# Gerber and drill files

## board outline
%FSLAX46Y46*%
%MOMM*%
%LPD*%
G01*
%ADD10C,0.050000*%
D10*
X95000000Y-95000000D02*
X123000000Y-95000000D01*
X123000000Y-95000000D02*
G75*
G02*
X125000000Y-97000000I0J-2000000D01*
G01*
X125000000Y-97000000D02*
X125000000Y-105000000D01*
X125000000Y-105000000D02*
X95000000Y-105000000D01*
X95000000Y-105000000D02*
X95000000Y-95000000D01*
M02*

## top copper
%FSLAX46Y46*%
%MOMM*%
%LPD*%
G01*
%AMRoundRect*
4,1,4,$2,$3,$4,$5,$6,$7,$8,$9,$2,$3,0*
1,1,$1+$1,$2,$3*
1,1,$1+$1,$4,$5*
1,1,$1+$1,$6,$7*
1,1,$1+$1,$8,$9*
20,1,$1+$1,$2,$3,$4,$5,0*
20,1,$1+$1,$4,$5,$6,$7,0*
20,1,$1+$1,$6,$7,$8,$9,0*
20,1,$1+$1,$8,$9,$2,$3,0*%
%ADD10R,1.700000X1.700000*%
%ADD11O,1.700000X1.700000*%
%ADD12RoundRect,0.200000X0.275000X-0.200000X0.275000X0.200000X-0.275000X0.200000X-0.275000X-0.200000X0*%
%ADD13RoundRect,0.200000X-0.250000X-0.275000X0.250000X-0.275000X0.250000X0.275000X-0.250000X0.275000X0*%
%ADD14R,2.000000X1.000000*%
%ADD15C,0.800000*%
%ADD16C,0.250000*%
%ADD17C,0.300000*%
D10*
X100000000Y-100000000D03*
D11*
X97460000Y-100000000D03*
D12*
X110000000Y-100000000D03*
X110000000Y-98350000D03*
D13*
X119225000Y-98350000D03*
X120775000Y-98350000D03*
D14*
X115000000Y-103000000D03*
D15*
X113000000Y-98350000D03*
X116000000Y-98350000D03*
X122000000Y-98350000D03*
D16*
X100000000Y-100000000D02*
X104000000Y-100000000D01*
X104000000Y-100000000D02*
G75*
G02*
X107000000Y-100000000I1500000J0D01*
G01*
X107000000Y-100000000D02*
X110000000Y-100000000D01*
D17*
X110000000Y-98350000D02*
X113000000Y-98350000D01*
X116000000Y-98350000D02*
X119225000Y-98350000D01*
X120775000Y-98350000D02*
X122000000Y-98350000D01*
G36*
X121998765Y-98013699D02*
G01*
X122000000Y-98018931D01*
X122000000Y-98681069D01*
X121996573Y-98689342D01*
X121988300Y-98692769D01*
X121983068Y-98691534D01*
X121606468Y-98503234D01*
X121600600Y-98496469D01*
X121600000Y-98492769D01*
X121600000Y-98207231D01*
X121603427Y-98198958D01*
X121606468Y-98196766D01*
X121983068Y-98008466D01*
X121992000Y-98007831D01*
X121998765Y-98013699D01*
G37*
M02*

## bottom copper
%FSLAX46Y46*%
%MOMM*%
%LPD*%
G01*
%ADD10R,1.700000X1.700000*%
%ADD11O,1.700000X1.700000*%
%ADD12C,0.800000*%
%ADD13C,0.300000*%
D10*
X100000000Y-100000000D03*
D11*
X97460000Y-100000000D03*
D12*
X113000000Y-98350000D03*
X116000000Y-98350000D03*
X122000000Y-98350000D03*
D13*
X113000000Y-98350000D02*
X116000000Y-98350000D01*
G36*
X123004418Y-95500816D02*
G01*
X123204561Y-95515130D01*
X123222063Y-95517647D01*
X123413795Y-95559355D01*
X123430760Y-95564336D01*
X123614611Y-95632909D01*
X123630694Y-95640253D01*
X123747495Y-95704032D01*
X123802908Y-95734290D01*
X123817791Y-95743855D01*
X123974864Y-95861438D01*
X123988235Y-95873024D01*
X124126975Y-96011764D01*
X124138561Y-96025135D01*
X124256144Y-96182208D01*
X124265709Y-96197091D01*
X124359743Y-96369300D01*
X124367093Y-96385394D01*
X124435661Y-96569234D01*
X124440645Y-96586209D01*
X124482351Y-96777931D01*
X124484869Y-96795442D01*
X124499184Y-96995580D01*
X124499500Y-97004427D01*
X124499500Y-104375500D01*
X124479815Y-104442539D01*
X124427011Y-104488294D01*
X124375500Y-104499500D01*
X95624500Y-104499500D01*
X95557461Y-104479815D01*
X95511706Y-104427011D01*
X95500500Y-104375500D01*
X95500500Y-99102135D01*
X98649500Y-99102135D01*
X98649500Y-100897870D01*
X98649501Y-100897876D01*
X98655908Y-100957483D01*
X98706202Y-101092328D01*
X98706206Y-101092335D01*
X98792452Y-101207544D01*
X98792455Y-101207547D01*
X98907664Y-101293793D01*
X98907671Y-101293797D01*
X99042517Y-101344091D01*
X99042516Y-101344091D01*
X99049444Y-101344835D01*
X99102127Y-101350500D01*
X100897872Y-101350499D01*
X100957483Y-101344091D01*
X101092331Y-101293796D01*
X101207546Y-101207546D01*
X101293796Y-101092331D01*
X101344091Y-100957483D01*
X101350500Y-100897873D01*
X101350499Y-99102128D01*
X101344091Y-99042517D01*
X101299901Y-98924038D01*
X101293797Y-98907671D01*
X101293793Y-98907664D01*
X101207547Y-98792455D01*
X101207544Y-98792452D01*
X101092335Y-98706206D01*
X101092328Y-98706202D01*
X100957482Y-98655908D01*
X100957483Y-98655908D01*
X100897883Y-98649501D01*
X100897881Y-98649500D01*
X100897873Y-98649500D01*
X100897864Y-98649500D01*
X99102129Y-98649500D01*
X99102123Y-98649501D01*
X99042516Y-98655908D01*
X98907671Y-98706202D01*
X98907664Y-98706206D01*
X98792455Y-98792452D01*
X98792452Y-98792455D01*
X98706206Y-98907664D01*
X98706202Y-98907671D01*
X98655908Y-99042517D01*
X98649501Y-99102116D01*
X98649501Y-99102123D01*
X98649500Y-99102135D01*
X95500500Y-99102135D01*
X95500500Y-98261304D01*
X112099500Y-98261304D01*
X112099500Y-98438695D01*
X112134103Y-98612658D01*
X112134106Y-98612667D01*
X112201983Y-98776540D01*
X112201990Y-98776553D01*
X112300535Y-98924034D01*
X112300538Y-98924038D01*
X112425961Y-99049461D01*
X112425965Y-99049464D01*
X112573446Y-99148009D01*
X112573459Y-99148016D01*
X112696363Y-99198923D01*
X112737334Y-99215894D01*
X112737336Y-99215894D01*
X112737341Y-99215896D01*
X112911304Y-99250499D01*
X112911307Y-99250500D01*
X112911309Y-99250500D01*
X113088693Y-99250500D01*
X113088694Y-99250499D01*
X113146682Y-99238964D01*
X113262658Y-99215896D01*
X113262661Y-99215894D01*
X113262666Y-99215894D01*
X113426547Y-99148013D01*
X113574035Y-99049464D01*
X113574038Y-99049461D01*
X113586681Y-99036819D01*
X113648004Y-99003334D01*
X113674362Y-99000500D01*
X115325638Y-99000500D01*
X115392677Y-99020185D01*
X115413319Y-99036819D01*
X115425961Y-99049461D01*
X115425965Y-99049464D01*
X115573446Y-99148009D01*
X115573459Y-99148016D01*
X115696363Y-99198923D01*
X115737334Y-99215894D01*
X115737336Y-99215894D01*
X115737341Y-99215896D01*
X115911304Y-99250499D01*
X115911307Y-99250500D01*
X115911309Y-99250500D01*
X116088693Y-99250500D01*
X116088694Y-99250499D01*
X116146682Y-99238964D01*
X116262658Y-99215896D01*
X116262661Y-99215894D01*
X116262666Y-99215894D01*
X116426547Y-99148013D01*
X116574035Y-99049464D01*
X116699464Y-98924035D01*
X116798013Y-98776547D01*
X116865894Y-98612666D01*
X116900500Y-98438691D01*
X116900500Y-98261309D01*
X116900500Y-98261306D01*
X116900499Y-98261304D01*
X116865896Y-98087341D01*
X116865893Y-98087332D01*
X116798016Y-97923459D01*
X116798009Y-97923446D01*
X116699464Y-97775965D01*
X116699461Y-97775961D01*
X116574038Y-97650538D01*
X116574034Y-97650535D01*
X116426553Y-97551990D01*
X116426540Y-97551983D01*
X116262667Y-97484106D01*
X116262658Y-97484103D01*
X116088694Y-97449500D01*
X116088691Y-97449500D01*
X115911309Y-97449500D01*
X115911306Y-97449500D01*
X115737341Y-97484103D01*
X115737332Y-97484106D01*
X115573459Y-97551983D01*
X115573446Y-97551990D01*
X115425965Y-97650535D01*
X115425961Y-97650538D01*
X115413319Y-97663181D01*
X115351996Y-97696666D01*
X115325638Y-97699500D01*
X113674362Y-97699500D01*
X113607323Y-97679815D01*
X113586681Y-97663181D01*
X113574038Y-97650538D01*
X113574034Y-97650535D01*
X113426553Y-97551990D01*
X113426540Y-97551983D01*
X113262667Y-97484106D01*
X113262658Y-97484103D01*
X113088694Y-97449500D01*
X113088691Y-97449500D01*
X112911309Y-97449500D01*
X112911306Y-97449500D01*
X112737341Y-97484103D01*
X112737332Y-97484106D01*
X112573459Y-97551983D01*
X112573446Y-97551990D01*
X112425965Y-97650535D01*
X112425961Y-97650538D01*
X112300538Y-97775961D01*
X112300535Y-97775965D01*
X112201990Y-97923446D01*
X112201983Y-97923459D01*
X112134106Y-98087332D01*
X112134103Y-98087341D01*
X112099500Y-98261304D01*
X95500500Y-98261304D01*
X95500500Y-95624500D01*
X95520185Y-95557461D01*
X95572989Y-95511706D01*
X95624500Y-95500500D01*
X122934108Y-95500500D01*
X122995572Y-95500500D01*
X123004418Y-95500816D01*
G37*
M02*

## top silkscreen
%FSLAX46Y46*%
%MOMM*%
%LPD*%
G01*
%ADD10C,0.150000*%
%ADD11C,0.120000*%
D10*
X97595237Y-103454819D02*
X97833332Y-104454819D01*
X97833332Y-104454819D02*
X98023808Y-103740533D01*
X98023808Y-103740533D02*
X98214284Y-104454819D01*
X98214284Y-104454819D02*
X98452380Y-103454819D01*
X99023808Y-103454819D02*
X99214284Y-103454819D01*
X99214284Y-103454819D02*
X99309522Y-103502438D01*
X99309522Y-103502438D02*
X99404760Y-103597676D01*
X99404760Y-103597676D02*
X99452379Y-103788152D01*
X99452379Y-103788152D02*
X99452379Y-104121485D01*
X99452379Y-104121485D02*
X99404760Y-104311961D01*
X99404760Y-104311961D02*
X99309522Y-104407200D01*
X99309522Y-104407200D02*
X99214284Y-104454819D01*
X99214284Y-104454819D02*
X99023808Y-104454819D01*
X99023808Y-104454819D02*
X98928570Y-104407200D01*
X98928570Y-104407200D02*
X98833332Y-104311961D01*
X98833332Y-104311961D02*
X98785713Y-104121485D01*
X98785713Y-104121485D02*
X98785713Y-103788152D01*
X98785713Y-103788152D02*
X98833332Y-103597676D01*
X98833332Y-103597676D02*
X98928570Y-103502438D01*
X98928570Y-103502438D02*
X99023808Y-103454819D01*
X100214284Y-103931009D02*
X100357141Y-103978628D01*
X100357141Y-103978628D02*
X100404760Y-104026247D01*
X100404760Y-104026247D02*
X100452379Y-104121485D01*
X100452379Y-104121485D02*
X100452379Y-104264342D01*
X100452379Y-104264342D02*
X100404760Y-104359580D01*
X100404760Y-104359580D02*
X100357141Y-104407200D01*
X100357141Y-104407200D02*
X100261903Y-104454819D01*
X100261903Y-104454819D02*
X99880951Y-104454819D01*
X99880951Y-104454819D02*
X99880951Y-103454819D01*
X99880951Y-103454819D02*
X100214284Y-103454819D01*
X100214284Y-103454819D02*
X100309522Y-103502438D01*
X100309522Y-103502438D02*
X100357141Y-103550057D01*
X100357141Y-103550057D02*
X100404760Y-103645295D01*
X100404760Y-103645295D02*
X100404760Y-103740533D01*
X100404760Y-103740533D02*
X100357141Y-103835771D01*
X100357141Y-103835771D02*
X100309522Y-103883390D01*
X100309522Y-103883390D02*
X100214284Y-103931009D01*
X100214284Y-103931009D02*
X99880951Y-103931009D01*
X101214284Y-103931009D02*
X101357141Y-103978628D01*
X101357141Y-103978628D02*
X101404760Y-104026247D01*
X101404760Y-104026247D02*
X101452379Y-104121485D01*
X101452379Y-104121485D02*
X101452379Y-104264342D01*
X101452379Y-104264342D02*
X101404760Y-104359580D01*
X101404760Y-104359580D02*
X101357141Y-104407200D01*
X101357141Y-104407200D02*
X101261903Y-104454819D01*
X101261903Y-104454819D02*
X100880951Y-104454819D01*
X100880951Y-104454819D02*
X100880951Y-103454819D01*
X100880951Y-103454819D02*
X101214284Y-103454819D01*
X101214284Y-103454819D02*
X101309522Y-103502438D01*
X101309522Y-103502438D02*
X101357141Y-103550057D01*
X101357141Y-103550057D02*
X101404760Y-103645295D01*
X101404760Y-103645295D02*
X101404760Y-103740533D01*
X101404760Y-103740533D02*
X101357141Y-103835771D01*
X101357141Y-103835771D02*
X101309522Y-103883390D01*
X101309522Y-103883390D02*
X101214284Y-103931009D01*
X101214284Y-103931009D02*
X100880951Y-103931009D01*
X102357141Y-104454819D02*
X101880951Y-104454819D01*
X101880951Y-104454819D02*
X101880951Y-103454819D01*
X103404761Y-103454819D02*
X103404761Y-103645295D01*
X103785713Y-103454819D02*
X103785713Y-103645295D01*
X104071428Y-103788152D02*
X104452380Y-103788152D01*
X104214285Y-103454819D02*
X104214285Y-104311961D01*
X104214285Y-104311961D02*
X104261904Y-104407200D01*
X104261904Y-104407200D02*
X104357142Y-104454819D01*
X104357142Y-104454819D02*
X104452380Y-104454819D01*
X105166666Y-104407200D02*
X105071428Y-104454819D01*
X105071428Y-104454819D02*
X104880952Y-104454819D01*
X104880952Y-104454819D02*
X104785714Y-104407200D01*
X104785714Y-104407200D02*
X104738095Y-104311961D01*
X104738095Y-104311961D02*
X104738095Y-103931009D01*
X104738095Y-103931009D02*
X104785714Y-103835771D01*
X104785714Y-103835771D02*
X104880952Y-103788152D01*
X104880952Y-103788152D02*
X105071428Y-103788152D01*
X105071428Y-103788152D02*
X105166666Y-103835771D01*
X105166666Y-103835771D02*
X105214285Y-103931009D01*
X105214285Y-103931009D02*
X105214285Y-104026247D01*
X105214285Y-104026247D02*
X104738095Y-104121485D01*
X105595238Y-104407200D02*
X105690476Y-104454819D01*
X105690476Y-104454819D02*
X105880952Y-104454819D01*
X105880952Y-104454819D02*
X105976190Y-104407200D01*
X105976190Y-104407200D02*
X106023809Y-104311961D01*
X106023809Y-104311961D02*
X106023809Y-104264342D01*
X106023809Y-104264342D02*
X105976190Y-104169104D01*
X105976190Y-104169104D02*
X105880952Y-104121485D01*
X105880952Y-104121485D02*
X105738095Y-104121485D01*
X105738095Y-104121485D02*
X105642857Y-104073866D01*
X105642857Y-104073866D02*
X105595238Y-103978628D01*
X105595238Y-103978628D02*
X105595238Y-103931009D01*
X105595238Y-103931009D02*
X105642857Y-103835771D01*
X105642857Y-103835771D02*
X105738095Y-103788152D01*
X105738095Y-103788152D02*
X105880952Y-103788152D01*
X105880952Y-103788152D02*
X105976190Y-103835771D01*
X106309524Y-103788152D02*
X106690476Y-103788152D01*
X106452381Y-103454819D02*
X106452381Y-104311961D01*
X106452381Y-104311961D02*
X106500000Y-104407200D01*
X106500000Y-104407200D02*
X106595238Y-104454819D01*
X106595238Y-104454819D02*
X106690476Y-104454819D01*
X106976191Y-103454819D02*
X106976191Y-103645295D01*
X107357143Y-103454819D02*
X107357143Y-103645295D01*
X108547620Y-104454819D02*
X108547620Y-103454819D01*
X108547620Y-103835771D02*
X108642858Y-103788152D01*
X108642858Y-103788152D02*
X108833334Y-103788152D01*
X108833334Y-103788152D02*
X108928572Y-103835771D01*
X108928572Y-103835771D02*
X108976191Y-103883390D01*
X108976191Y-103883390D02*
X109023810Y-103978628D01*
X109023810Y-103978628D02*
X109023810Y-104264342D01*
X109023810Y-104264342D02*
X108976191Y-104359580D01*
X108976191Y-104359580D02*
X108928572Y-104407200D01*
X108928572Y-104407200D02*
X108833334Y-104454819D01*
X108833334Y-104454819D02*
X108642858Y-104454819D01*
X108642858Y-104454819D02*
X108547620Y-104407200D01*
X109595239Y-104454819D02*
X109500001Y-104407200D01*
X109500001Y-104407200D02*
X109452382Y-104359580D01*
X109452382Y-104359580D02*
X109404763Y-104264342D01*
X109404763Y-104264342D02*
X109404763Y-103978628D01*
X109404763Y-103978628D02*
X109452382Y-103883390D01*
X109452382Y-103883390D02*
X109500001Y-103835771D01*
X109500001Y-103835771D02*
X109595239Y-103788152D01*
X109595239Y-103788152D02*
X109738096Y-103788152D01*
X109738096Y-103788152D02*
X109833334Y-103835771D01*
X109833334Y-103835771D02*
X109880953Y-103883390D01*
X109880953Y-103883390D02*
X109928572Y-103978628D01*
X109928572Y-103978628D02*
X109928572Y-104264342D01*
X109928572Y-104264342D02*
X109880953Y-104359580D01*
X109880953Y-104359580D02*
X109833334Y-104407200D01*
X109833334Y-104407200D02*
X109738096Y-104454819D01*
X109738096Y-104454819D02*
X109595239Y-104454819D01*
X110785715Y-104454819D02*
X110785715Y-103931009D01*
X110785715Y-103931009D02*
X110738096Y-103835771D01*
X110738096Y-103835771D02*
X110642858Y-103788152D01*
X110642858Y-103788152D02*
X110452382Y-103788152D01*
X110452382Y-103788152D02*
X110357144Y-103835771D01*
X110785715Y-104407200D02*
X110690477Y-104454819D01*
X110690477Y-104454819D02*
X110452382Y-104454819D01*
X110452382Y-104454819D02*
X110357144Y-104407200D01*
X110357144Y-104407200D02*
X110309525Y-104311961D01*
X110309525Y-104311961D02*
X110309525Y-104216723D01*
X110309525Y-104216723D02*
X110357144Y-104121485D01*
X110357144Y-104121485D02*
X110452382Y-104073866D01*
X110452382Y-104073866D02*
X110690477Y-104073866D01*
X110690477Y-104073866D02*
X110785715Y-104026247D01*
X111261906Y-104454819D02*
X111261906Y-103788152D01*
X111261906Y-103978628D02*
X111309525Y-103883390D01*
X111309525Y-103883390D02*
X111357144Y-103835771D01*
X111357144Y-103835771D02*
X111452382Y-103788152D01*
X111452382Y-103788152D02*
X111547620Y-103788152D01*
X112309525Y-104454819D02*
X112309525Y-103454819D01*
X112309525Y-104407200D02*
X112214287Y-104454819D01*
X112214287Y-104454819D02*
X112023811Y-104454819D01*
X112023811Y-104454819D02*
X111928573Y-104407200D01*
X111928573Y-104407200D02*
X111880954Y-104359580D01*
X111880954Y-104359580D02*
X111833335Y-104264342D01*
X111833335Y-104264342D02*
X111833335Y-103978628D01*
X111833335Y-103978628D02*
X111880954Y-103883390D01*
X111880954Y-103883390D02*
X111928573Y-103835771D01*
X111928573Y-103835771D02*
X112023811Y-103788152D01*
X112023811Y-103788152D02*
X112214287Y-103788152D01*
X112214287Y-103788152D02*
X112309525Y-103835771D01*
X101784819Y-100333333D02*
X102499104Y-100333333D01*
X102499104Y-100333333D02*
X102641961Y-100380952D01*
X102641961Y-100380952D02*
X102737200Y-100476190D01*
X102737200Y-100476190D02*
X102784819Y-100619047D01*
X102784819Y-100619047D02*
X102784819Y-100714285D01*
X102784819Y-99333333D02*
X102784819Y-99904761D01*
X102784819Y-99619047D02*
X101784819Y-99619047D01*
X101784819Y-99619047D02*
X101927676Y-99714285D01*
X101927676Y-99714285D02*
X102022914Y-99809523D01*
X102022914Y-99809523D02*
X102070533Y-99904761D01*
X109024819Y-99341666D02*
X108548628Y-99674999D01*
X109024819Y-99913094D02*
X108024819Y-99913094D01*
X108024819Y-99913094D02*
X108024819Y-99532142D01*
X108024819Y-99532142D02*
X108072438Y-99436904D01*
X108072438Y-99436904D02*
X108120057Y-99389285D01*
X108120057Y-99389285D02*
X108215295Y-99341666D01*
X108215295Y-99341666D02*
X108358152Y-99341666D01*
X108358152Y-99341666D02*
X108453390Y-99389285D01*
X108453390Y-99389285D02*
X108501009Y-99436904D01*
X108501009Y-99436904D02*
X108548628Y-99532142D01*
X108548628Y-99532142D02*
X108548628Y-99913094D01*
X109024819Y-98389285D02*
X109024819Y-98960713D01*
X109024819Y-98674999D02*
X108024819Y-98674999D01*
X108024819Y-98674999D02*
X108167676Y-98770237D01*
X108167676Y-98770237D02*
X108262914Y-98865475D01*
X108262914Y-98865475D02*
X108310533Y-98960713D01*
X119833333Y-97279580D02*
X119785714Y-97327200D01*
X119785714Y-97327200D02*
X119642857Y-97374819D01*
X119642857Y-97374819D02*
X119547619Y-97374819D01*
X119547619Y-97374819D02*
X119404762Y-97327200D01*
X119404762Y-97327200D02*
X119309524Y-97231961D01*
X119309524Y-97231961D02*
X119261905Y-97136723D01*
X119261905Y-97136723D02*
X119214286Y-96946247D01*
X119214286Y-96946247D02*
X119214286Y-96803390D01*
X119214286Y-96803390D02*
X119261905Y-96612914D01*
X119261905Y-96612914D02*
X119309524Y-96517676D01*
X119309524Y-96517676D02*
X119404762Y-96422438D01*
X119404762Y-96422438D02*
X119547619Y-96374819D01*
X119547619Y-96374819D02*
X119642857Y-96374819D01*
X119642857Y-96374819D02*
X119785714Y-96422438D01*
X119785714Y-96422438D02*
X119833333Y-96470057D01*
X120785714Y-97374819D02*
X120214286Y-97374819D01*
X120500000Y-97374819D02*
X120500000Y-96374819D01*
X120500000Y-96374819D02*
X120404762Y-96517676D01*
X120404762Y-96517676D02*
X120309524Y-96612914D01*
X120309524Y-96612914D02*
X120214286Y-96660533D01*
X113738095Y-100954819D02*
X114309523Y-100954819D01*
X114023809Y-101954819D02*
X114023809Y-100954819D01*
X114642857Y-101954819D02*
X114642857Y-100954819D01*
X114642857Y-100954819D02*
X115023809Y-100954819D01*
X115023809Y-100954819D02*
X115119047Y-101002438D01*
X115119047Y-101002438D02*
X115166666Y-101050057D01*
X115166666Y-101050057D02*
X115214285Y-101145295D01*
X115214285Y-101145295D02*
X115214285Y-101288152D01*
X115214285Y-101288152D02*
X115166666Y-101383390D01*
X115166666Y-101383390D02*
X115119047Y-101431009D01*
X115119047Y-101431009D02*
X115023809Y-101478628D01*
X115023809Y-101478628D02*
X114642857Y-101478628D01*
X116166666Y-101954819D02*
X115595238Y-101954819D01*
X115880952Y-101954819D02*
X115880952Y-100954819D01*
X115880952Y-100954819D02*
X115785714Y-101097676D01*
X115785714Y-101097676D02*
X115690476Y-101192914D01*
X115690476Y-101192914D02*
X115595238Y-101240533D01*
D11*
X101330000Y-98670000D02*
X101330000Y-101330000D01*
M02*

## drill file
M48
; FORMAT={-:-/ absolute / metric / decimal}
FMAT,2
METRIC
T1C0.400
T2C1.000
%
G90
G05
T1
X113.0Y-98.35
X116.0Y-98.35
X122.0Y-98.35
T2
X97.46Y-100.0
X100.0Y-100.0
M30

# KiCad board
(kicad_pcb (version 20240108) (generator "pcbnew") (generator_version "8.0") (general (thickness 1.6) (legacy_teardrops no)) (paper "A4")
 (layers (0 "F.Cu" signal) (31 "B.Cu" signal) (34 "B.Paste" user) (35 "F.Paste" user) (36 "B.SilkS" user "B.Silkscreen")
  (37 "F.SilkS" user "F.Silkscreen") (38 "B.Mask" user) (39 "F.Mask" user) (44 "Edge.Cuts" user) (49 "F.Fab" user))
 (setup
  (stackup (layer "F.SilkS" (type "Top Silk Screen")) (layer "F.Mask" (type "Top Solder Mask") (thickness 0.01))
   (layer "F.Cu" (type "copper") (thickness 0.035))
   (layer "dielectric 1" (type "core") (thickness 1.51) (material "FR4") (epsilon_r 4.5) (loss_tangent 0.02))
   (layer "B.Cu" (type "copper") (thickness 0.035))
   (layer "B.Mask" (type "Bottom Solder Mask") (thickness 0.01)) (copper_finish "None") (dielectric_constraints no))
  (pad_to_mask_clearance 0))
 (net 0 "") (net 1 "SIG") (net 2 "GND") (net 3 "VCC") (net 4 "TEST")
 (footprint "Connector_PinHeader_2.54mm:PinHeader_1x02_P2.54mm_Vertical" (layer "F.Cu") (at 100 100 270)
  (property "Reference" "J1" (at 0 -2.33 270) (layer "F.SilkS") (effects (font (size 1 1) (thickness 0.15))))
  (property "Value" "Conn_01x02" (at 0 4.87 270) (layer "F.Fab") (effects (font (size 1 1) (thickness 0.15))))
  (fp_line (start -1.33 -1.33) (end 1.33 -1.33) (stroke (width 0.12) (type solid)) (layer "F.SilkS"))
  (pad "1" thru_hole rect (at 0 0 270) (size 1.7 1.7) (drill 1) (layers "*.Cu" "*.Mask") (remove_unused_layers no) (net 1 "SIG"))
  (pad "2" thru_hole oval (at 0 2.54 270) (size 1.7 1.7) (drill 1) (layers "*.Cu" "*.Mask") (remove_unused_layers no) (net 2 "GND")))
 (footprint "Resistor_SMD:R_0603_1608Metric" (layer "F.Cu") (at 110 99.175 90)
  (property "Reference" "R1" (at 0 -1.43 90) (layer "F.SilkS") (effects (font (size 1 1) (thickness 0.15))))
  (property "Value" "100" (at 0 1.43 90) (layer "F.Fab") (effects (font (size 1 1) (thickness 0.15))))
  (pad "1" smd roundrect (at -0.825 0 90) (size 0.8 0.95) (layers "F.Cu" "F.Paste" "F.Mask") (roundrect_rratio 0.25) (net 1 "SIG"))
  (pad "2" smd roundrect (at 0.825 0 90) (size 0.8 0.95) (layers "F.Cu" "F.Paste" "F.Mask") (roundrect_rratio 0.25) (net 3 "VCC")))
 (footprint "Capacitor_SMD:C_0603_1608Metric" (layer "F.Cu") (at 120 98.35)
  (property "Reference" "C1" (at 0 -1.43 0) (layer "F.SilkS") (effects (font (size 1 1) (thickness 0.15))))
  (pad "1" smd roundrect (at -0.775 0) (size 0.9 0.95) (layers "F.Cu" "F.Paste" "F.Mask") (roundrect_rratio 0.222222) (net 3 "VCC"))
  (pad "2" smd roundrect (at 0.775 0) (size 0.9 0.95) (layers "F.Cu" "F.Paste" "F.Mask") (roundrect_rratio 0.222222) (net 2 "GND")))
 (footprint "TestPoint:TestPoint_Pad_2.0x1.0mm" (layer "F.Cu") (at 115 103)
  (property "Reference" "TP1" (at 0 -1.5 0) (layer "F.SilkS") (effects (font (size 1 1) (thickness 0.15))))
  (pad "1" smd rect (at 0 0) (size 2 1) (layers "F.Cu" "F.Mask") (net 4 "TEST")))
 (gr_line (start 95 95) (end 123 95) (stroke (width 0.05) (type default)) (layer "Edge.Cuts"))
 (gr_arc (start 123 95) (mid 124.414214 95.585786) (end 125 97) (stroke (width 0.05) (type default)) (layer "Edge.Cuts"))
 (gr_line (start 125 97) (end 125 105) (stroke (width 0.05) (type default)) (layer "Edge.Cuts"))
 (gr_line (start 125 105) (end 95 105) (stroke (width 0.05) (type default)) (layer "Edge.Cuts"))
 (gr_line (start 95 105) (end 95 95) (stroke (width 0.05) (type default)) (layer "Edge.Cuts"))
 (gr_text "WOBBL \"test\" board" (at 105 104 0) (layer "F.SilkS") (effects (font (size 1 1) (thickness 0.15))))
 (segment (start 100 100) (end 104 100) (width 0.25) (layer "F.Cu") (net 1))
 (arc (start 104 100) (mid 105.5 98.5) (end 107 100) (width 0.25) (layer "F.Cu") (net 1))
 (segment (start 107 100) (end 110 100) (width 0.25) (layer "F.Cu") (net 1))
 (segment (start 110 98.35) (end 113 98.35) (width 0.3) (layer "F.Cu") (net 3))
 (segment (start 113 98.35) (end 116 98.35) (width 0.3) (layer "B.Cu") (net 3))
 (segment (start 116 98.35) (end 119.225 98.35) (width 0.3) (layer "F.Cu") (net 3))
 (segment (start 120.775 98.35) (end 122 98.35) (width 0.3) (layer "F.Cu") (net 2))
 (via (at 113 98.35) (size 0.8) (drill 0.4) (layers "F.Cu" "B.Cu") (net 3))
 (via (at 116 98.35) (size 0.8) (drill 0.4) (layers "F.Cu" "B.Cu") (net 3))
 (via (at 122 98.35) (size 0.8) (drill 0.4) (layers "F.Cu" "B.Cu") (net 2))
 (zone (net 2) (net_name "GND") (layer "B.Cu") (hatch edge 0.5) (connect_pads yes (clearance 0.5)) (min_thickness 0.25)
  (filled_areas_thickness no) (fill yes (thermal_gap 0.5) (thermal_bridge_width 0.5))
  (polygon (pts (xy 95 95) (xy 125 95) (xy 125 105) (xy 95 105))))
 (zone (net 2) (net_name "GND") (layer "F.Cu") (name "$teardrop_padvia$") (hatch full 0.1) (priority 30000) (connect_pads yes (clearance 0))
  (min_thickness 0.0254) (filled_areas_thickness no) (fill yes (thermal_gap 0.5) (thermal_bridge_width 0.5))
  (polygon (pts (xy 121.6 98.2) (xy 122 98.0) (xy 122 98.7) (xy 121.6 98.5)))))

